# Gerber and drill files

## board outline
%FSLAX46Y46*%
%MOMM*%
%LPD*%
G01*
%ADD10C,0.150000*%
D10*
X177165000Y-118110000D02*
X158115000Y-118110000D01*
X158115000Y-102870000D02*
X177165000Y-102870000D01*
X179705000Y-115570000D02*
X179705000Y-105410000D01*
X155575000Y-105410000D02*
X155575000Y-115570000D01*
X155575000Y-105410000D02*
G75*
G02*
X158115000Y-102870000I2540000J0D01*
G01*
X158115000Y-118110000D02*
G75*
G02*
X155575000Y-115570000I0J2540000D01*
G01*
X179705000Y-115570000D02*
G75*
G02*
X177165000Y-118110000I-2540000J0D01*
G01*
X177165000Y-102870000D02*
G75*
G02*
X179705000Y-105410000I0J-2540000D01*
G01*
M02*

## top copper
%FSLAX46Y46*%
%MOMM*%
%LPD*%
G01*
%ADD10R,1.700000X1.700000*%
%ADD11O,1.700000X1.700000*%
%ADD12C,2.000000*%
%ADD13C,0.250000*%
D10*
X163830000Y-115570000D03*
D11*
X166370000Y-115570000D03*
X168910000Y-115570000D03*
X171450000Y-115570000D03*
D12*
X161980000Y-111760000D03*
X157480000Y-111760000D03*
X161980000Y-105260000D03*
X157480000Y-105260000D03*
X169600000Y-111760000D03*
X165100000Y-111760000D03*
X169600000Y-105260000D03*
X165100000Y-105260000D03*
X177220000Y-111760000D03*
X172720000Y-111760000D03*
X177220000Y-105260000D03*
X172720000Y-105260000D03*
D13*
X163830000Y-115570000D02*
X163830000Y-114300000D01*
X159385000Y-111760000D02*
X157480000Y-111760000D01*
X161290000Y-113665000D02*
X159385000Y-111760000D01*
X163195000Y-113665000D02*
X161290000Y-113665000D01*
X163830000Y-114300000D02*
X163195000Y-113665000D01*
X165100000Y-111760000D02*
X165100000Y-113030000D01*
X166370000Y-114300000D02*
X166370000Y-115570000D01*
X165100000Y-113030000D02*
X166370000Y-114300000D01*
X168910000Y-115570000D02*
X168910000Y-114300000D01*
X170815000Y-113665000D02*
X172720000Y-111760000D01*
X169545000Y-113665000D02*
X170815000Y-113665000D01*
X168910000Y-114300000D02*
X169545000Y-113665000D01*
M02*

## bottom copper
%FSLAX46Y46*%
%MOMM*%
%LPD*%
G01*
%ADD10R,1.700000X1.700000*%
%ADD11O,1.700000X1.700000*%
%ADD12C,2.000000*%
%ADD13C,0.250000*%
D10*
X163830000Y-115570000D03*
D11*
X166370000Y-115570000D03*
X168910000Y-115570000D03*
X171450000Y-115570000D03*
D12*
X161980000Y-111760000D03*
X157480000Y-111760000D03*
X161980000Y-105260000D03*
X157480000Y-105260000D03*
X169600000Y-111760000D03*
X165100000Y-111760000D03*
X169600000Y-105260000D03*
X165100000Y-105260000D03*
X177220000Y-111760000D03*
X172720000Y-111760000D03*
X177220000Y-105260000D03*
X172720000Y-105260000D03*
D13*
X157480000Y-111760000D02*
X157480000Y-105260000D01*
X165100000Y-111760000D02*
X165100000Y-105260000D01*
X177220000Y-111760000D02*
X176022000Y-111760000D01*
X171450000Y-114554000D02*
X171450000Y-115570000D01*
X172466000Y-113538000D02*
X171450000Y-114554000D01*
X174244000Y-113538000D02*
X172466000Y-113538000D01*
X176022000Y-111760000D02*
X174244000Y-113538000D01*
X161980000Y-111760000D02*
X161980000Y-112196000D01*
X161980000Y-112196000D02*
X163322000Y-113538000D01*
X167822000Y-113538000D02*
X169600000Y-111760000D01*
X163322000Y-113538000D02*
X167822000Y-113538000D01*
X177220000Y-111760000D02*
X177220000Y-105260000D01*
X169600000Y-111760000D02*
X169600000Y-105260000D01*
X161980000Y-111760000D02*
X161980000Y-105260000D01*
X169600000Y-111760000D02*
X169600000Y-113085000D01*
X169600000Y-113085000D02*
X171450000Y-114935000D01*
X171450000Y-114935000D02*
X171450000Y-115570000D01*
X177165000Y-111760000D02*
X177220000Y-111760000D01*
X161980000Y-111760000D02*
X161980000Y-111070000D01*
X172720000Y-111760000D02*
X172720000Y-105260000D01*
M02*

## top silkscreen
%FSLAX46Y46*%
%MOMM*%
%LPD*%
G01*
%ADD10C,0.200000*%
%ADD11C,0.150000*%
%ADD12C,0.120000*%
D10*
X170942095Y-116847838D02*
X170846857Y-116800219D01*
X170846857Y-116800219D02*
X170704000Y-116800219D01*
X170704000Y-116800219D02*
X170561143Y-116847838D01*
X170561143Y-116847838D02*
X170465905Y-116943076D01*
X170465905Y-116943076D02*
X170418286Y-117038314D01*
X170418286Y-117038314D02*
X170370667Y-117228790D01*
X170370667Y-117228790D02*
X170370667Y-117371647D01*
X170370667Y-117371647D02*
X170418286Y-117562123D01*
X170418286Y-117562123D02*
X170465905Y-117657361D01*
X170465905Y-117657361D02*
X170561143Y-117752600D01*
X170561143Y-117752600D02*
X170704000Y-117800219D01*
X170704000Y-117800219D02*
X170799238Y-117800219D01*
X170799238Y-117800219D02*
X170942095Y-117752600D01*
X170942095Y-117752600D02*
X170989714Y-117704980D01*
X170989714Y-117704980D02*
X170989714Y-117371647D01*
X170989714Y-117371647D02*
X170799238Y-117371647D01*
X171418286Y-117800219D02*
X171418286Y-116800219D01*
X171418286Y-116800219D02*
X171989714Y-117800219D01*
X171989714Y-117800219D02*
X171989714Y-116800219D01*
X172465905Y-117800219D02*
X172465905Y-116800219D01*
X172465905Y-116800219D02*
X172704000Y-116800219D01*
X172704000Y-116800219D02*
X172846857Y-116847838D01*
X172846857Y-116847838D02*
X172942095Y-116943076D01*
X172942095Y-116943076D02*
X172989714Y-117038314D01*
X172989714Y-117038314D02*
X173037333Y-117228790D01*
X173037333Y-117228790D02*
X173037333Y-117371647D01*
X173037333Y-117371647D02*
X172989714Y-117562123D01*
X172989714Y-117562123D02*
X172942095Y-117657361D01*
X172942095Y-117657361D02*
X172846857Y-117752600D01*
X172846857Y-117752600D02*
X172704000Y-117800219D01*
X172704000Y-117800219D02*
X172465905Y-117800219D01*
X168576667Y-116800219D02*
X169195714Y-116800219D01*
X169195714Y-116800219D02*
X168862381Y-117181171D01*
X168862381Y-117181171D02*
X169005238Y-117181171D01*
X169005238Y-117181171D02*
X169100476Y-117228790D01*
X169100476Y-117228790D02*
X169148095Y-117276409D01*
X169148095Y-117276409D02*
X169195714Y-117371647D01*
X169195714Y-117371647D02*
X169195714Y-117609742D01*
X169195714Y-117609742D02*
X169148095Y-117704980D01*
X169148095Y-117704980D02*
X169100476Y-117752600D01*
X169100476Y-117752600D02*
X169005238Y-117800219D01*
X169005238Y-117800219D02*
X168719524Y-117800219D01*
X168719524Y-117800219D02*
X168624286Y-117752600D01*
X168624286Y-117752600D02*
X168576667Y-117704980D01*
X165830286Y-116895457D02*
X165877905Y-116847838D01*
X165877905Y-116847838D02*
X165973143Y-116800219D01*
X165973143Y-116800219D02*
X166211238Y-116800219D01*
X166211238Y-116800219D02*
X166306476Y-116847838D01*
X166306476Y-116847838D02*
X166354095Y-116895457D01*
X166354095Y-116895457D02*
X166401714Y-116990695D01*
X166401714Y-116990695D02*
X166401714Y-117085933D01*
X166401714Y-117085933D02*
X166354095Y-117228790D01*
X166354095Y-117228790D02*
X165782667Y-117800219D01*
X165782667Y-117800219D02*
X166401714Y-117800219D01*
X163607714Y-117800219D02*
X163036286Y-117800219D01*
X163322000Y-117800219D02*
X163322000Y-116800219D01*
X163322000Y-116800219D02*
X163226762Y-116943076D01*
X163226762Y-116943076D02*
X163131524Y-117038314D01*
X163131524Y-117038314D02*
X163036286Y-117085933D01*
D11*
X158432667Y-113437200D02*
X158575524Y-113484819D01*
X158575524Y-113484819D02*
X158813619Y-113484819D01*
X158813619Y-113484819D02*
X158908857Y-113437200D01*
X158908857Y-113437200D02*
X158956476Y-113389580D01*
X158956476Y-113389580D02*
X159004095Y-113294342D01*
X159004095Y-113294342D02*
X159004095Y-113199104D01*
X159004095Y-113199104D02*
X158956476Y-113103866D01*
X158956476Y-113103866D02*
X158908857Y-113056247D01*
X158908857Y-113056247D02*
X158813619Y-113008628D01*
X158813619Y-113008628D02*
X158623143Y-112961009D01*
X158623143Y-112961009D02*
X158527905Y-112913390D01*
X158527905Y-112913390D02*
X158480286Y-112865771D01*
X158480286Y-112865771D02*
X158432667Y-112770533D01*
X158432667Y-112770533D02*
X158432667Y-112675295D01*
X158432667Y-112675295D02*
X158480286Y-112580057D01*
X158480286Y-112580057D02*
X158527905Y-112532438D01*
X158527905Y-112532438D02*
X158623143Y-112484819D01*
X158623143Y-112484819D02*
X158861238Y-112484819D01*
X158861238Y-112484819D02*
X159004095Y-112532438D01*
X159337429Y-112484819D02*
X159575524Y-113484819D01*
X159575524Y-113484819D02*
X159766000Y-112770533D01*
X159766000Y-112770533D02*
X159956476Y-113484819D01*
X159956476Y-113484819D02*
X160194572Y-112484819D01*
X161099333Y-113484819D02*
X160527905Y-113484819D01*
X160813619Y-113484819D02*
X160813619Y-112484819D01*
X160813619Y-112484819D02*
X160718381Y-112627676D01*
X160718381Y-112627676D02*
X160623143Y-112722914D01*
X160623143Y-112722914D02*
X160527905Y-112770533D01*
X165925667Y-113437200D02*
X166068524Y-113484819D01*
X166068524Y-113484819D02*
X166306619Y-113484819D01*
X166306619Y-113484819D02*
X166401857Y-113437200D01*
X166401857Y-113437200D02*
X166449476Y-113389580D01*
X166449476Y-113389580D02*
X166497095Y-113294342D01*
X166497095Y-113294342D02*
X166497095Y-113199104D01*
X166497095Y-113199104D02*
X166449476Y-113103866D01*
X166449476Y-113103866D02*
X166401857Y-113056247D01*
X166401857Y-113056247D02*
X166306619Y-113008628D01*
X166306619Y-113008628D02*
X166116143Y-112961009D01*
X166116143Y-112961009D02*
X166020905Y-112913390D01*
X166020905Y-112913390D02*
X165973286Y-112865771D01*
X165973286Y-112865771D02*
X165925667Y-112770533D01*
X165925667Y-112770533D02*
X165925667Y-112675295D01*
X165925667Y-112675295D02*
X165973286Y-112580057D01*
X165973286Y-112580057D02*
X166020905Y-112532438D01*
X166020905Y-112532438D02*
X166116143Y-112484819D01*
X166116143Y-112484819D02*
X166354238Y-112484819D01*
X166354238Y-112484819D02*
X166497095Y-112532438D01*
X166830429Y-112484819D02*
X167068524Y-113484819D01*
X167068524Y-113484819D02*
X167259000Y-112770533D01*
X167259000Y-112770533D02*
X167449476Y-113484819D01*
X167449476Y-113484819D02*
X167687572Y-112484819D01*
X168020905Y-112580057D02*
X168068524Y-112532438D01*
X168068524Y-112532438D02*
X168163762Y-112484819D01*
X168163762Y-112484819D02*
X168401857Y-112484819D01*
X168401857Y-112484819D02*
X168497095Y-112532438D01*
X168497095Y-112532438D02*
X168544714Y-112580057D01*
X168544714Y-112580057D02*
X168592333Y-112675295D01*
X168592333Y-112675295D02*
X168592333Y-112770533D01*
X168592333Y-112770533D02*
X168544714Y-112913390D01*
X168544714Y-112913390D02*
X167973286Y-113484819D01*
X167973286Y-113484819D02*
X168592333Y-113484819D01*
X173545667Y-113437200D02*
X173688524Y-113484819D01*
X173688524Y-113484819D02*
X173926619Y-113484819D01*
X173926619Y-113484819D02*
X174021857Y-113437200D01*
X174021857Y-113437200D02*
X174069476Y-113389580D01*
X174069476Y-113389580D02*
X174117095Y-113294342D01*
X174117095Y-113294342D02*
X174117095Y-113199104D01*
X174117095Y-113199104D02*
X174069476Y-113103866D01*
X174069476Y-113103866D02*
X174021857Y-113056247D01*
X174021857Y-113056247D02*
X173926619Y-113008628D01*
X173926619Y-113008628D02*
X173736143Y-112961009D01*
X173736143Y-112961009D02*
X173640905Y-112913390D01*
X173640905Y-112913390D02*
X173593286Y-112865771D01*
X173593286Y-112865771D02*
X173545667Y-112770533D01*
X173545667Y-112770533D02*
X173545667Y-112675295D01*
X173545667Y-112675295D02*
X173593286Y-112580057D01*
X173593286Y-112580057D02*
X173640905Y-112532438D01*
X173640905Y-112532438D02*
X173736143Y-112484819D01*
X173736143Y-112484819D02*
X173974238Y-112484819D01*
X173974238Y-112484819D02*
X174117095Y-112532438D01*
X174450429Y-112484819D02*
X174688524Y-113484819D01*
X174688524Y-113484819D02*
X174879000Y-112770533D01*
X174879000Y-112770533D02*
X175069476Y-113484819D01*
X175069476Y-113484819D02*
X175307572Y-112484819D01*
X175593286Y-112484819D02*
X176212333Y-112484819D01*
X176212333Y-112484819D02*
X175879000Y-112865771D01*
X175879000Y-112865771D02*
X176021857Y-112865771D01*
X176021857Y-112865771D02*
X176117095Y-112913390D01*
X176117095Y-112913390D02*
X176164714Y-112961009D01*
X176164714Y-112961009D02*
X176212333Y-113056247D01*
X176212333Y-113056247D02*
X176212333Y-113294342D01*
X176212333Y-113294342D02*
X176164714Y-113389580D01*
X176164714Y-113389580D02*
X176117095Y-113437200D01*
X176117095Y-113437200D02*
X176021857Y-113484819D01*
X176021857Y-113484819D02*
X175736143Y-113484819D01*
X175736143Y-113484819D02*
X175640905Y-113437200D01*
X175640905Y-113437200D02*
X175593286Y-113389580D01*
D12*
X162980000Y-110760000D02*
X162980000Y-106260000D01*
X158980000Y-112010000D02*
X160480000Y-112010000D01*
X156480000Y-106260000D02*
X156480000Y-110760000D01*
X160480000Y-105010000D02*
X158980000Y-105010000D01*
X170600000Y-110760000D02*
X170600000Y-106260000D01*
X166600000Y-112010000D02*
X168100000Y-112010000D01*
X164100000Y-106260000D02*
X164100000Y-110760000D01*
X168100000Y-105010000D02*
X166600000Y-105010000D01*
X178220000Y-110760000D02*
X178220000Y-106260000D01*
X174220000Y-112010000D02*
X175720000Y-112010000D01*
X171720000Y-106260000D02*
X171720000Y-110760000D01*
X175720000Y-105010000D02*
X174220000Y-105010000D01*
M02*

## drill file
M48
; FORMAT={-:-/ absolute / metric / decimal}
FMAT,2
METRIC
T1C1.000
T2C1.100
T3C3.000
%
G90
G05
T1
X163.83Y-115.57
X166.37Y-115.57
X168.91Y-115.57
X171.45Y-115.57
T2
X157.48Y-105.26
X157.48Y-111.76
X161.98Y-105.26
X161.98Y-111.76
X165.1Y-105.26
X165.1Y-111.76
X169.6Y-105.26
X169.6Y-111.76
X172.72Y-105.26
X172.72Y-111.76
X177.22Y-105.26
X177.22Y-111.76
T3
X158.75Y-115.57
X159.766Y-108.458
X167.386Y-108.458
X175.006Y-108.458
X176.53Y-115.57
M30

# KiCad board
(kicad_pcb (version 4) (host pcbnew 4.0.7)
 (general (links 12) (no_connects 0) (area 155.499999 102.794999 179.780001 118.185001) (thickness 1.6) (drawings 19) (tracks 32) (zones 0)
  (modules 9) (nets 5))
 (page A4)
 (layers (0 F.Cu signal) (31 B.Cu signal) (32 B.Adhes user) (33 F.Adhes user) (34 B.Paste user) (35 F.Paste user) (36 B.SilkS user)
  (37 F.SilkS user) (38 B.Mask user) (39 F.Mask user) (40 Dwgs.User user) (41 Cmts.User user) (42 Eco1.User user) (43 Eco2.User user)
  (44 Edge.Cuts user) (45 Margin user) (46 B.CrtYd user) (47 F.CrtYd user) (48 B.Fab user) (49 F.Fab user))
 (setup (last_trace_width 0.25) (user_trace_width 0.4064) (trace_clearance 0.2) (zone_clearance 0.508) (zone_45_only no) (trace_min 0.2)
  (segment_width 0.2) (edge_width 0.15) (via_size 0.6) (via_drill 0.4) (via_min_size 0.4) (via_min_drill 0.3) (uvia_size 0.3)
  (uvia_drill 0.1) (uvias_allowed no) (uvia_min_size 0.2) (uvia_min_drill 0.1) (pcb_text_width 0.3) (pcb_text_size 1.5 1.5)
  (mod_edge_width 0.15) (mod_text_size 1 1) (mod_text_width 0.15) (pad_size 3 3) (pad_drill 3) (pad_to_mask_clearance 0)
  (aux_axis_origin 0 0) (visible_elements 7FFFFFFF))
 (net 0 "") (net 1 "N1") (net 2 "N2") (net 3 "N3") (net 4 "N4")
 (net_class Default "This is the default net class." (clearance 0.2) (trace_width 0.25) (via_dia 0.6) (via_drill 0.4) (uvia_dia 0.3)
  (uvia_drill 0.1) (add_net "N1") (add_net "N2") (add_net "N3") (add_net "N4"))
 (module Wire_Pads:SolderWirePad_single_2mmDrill (layer F.Cu) (at 175.006 108.458)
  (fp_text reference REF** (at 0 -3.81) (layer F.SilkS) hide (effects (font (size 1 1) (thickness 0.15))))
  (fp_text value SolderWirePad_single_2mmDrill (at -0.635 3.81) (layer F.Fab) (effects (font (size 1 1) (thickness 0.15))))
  (pad "" np_thru_hole circle (at 0 0) (size 3 3) (drill 3) (layers *.Cu *.Mask)))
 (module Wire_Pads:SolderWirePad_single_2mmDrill (layer F.Cu) (at 167.386 108.458)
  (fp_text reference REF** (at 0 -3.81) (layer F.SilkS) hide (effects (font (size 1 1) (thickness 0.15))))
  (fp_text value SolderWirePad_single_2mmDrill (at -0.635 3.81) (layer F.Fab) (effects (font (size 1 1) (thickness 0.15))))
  (pad "" np_thru_hole circle (at 0 0) (size 3 3) (drill 3) (layers *.Cu *.Mask)))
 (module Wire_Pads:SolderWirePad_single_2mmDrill (layer F.Cu) (at 159.766 108.458)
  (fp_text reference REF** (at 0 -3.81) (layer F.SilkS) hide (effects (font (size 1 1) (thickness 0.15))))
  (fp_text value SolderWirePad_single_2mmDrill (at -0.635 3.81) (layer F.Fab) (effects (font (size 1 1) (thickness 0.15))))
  (pad "" np_thru_hole circle (at 0 0) (size 3 3) (drill 3) (layers *.Cu *.Mask)))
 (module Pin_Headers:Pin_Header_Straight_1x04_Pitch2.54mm (layer F.Cu) (at 163.83 115.57 90)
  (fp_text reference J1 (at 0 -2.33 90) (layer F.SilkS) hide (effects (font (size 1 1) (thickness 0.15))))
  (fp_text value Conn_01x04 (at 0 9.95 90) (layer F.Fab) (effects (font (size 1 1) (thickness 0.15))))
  (pad 1 thru_hole rect (at 0 0 90) (size 1.7 1.7) (drill 1) (layers *.Cu *.Mask) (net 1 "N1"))
  (pad 2 thru_hole oval (at 0 2.54 90) (size 1.7 1.7) (drill 1) (layers *.Cu *.Mask) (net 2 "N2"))
  (pad 3 thru_hole oval (at 0 5.08 90) (size 1.7 1.7) (drill 1) (layers *.Cu *.Mask) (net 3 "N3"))
  (pad 4 thru_hole oval (at 0 7.62 90) (size 1.7 1.7) (drill 1) (layers *.Cu *.Mask) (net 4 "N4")))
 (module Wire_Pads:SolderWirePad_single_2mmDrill (layer F.Cu) (at 158.75 115.57)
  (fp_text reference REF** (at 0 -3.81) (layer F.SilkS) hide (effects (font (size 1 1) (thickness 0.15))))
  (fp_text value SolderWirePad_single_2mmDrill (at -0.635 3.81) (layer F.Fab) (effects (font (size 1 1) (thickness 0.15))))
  (pad "" np_thru_hole circle (at 0 0) (size 3 3) (drill 3) (layers *.Cu *.Mask)))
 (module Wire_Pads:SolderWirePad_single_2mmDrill (layer F.Cu) (at 176.53 115.57)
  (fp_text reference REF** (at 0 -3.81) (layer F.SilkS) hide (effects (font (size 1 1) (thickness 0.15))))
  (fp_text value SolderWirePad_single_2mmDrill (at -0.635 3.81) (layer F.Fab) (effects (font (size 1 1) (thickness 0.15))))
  (pad "" np_thru_hole circle (at 0 0) (size 3 3) (drill 3) (layers *.Cu *.Mask)))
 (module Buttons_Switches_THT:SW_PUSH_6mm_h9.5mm (layer F.Cu) (at 157.48 111.76 90)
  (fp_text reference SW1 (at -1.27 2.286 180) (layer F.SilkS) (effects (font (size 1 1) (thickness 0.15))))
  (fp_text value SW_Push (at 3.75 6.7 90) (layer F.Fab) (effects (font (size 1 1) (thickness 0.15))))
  (fp_line (start 1 5.5) (end 5.5 5.5) (layer F.SilkS) (width 0.12))
  (fp_line (start -0.25 1.5) (end -0.25 3) (layer F.SilkS) (width 0.12))
  (fp_line (start 5.5 -1) (end 1 -1) (layer F.SilkS) (width 0.12))
  (fp_line (start 6.75 3) (end 6.75 1.5) (layer F.SilkS) (width 0.12))
  (pad 2 thru_hole circle (at 0 4.5 180) (size 2 2) (drill 1.1) (layers *.Cu *.Mask) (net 4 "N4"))
  (pad 1 thru_hole circle (at 0 0 180) (size 2 2) (drill 1.1) (layers *.Cu *.Mask) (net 1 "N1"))
  (pad 2 thru_hole circle (at 6.5 4.5 180) (size 2 2) (drill 1.1) (layers *.Cu *.Mask) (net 4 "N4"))
  (pad 1 thru_hole circle (at 6.5 0 180) (size 2 2) (drill 1.1) (layers *.Cu *.Mask) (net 1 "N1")))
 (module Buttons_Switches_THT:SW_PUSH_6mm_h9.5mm (layer F.Cu) (at 165.1 111.76 90)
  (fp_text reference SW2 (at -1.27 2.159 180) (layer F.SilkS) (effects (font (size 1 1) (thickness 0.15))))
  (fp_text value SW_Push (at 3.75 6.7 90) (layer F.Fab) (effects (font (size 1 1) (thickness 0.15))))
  (fp_line (start 1 5.5) (end 5.5 5.5) (layer F.SilkS) (width 0.12))
  (fp_line (start -0.25 1.5) (end -0.25 3) (layer F.SilkS) (width 0.12))
  (fp_line (start 5.5 -1) (end 1 -1) (layer F.SilkS) (width 0.12))
  (fp_line (start 6.75 3) (end 6.75 1.5) (layer F.SilkS) (width 0.12))
  (pad 2 thru_hole circle (at 0 4.5 180) (size 2 2) (drill 1.1) (layers *.Cu *.Mask) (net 4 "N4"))
  (pad 1 thru_hole circle (at 0 0 180) (size 2 2) (drill 1.1) (layers *.Cu *.Mask) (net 2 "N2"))
  (pad 2 thru_hole circle (at 6.5 4.5 180) (size 2 2) (drill 1.1) (layers *.Cu *.Mask) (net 4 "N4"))
  (pad 1 thru_hole circle (at 6.5 0 180) (size 2 2) (drill 1.1) (layers *.Cu *.Mask) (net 2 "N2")))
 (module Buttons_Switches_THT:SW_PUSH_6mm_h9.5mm (layer F.Cu) (at 172.72 111.76 90)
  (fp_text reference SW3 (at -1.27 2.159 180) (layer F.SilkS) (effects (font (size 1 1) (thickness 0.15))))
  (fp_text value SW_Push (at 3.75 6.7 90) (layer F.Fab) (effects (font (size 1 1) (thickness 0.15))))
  (fp_line (start 1 5.5) (end 5.5 5.5) (layer F.SilkS) (width 0.12))
  (fp_line (start -0.25 1.5) (end -0.25 3) (layer F.SilkS) (width 0.12))
  (fp_line (start 5.5 -1) (end 1 -1) (layer F.SilkS) (width 0.12))
  (fp_line (start 6.75 3) (end 6.75 1.5) (layer F.SilkS) (width 0.12))
  (pad 2 thru_hole circle (at 0 4.5 180) (size 2 2) (drill 1.1) (layers *.Cu *.Mask) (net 4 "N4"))
  (pad 1 thru_hole circle (at 0 0 180) (size 2 2) (drill 1.1) (layers *.Cu *.Mask) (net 3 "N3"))
  (pad 2 thru_hole circle (at 6.5 4.5 180) (size 2 2) (drill 1.1) (layers *.Cu *.Mask) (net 4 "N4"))
  (pad 1 thru_hole circle (at 6.5 0 180) (size 2 2) (drill 1.1) (layers *.Cu *.Mask) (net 3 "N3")))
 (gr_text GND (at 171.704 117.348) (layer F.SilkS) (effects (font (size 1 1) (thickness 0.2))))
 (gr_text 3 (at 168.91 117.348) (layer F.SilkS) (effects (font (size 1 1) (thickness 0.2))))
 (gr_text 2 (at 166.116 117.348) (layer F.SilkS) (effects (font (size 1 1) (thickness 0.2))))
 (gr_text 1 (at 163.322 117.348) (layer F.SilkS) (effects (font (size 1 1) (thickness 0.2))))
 (gr_line (start 177.165 118.11) (end 158.115 118.11) (angle 90) (layer Edge.Cuts) (width 0.15))
 (gr_line (start 158.115 102.87) (end 177.165 102.87) (angle 90) (layer Edge.Cuts) (width 0.15))
 (gr_line (start 179.705 115.57) (end 179.705 105.41) (angle 90) (layer Edge.Cuts) (width 0.15))
 (gr_line (start 155.575 105.41) (end 155.575 115.57) (angle 90) (layer Edge.Cuts) (width 0.15))
 (gr_arc (start 158.115 105.41) (end 155.575 105.41) (angle 90) (layer Edge.Cuts) (width 0.15))
 (gr_arc (start 158.115 115.57) (end 158.115 118.11) (angle 90) (layer Edge.Cuts) (width 0.15))
 (gr_arc (start 177.165 115.57) (end 179.705 115.57) (angle 90) (layer Edge.Cuts) (width 0.15))
 (gr_arc (start 177.165 105.41) (end 177.165 102.87) (angle 90) (layer Edge.Cuts) (width 0.15))
 (segment (start 157.48 111.76) (end 157.48 105.26) (width 0.25) (layer B.Cu) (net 1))
 (segment (start 163.83 115.57) (end 163.83 114.3) (width 0.25) (layer F.Cu) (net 1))
 (segment (start 159.385 111.76) (end 157.48 111.76) (width 0.25) (layer F.Cu) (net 1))
 (segment (start 161.29 113.665) (end 159.385 111.76) (width 0.25) (layer F.Cu) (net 1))
 (segment (start 163.195 113.665) (end 161.29 113.665) (width 0.25) (layer F.Cu) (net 1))
 (segment (start 163.83 114.3) (end 163.195 113.665) (width 0.25) (layer F.Cu) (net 1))
 (segment (start 165.1 111.76) (end 165.1 105.26) (width 0.25) (layer B.Cu) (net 2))
 (segment (start 165.1 111.76) (end 165.1 113.03) (width 0.25) (layer F.Cu) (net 2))
 (segment (start 166.37 114.3) (end 166.37 115.57) (width 0.25) (layer F.Cu) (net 2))
 (segment (start 165.1 113.03) (end 166.37 114.3) (width 0.25) (layer F.Cu) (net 2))
 (segment (start 177.22 111.76) (end 176.022 111.76) (width 0.25) (layer B.Cu) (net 4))
 (segment (start 171.45 114.554) (end 171.45 115.57) (width 0.25) (layer B.Cu) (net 4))
 (segment (start 172.466 113.538) (end 171.45 114.554) (width 0.25) (layer B.Cu) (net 4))
 (segment (start 174.244 113.538) (end 172.466 113.538) (width 0.25) (layer B.Cu) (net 4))
 (segment (start 176.022 111.76) (end 174.244 113.538) (width 0.25) (layer B.Cu) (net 4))
 (segment (start 161.98 111.76) (end 161.98 112.196) (width 0.25) (layer B.Cu) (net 4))
 (segment (start 161.98 112.196) (end 163.322 113.538) (width 0.25) (layer B.Cu) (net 4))
 (segment (start 167.822 113.538) (end 169.6 111.76) (width 0.25) (layer B.Cu) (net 4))
 (segment (start 163.322 113.538) (end 167.822 113.538) (width 0.25) (layer B.Cu) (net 4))
 (segment (start 177.22 111.76) (end 177.22 105.26) (width 0.25) (layer B.Cu) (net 4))
 (segment (start 169.6 111.76) (end 169.6 105.26) (width 0.25) (layer B.Cu) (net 4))
 (segment (start 161.98 111.76) (end 161.98 105.26) (width 0.25) (layer B.Cu) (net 4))
 (segment (start 169.6 111.76) (end 169.6 113.085) (width 0.25) (layer B.Cu) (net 4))
 (segment (start 169.6 113.085) (end 171.45 114.935) (width 0.25) (layer B.Cu) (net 4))
 (segment (start 171.45 114.935) (end 171.45 115.57) (width 0.25) (layer B.Cu) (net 4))
 (segment (start 177.165 111.76) (end 177.22 111.76) (width 0.25) (layer B.Cu) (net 4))
 (segment (start 161.98 111.76) (end 161.98 111.07) (width 0.25) (layer B.Cu) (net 4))
 (segment (start 172.72 111.76) (end 172.72 105.26) (width 0.25) (layer B.Cu) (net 3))
 (segment (start 168.91 115.57) (end 168.91 114.3) (width 0.25) (layer F.Cu) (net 3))
 (segment (start 170.815 113.665) (end 172.72 111.76) (width 0.25) (layer F.Cu) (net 3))
 (segment (start 169.545 113.665) (end 170.815 113.665) (width 0.25) (layer F.Cu) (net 3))
 (segment (start 168.91 114.3) (end 169.545 113.665) (width 0.25) (layer F.Cu) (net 3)))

